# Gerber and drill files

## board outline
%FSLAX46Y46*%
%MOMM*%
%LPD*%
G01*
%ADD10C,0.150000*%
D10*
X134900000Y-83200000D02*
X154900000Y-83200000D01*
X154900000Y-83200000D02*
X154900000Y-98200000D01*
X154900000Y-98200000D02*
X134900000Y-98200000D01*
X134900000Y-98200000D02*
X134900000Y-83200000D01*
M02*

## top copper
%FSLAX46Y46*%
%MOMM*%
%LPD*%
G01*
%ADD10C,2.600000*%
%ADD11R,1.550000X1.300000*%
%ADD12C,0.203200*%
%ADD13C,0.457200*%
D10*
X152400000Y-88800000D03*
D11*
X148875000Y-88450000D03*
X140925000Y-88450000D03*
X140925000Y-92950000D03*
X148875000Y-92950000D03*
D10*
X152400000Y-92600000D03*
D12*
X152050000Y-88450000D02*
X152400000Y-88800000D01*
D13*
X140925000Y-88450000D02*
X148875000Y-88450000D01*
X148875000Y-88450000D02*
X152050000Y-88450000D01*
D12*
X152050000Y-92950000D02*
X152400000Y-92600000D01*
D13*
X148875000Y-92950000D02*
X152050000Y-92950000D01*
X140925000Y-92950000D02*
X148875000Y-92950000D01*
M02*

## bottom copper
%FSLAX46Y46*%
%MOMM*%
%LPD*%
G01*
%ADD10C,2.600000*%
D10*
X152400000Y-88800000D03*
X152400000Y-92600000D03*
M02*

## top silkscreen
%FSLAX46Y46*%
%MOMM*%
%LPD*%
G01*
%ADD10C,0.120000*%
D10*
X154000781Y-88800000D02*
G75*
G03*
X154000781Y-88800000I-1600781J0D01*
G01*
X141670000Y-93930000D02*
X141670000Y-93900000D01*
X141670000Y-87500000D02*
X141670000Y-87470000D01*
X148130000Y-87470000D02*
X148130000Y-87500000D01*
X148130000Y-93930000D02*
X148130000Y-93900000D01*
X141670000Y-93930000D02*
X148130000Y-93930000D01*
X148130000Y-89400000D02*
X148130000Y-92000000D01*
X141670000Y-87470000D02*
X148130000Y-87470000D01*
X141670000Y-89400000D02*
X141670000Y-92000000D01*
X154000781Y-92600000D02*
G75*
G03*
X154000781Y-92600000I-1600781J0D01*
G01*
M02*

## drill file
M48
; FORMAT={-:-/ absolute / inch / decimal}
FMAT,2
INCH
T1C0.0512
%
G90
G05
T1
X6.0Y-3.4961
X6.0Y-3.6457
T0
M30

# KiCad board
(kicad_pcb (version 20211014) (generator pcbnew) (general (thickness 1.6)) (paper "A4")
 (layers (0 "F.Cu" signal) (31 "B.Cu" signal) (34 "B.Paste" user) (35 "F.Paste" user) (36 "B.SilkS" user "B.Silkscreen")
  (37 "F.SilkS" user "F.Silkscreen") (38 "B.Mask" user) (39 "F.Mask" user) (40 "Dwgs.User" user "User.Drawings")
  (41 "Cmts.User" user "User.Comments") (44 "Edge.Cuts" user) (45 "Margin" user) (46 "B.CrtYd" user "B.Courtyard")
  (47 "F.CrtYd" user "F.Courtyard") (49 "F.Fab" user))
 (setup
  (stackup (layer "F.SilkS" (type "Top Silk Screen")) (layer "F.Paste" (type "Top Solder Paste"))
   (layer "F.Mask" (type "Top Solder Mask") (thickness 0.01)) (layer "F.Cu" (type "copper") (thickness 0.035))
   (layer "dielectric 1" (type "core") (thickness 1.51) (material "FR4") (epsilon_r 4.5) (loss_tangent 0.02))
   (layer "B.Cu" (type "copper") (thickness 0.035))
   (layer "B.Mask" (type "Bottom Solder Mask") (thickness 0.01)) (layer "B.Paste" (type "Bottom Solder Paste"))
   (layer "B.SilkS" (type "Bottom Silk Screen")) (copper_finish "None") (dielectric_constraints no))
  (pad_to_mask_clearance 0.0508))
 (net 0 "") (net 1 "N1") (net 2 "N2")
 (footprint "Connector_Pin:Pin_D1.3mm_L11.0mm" (layer "F.Cu") (at 152.4 88.8)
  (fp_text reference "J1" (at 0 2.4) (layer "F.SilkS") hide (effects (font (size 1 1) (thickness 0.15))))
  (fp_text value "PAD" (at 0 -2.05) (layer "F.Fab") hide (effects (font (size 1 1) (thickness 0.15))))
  (fp_circle (center 0 0) (end 1.6 0.05) (layer "F.SilkS") (width 0.12) (fill none))
  (pad "1" thru_hole circle (at 0 0) (size 2.6 2.6) (drill 1.3) (layers *.Cu *.Mask) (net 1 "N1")))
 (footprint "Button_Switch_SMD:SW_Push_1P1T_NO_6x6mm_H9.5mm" (layer "F.Cu") (at 144.9 90.7)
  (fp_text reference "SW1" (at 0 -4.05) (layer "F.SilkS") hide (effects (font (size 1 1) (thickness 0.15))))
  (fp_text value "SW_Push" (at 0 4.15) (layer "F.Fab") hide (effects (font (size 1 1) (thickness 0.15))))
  (fp_line (start -3.23 3.23) (end -3.23 3.2) (layer "F.SilkS") (width 0.12))
  (fp_line (start -3.23 -3.2) (end -3.23 -3.23) (layer "F.SilkS") (width 0.12))
  (fp_line (start 3.23 -3.23) (end 3.23 -3.2) (layer "F.SilkS") (width 0.12))
  (fp_line (start 3.23 3.23) (end 3.23 3.2) (layer "F.SilkS") (width 0.12))
  (fp_line (start -3.23 3.23) (end 3.23 3.23) (layer "F.SilkS") (width 0.12))
  (fp_line (start 3.23 -1.3) (end 3.23 1.3) (layer "F.SilkS") (width 0.12))
  (fp_line (start -3.23 -3.23) (end 3.23 -3.23) (layer "F.SilkS") (width 0.12))
  (fp_line (start -3.23 -1.3) (end -3.23 1.3) (layer "F.SilkS") (width 0.12))
  (pad "1" smd rect (at 3.975 -2.25) (size 1.55 1.3) (layers "F.Cu" "F.Paste" "F.Mask") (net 1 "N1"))
  (pad "1" smd rect (at -3.975 -2.25) (size 1.55 1.3) (layers "F.Cu" "F.Paste" "F.Mask") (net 1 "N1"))
  (pad "2" smd rect (at -3.975 2.25) (size 1.55 1.3) (layers "F.Cu" "F.Paste" "F.Mask") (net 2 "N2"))
  (pad "2" smd rect (at 3.975 2.25) (size 1.55 1.3) (layers "F.Cu" "F.Paste" "F.Mask") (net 2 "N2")))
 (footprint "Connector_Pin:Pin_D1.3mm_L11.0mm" (layer "F.Cu") (at 152.4 92.6)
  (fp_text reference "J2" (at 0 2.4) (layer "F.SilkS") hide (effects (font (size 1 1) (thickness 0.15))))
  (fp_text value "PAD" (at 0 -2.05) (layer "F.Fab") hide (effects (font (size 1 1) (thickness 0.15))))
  (fp_circle (center 0 0) (end 1.6 0.05) (layer "F.SilkS") (width 0.12) (fill none))
  (pad "1" thru_hole circle (at 0 0) (size 2.6 2.6) (drill 1.3) (layers *.Cu *.Mask) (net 2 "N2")))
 (gr_rect (start 134.9 83.2) (end 154.9 98.2) (layer "Edge.Cuts") (width 0.15) (fill none))
 (segment (start 152.05 88.45) (end 152.4 88.8) (width 0.2032) (layer "F.Cu") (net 1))
 (segment (start 140.925 88.45) (end 148.875 88.45) (width 0.4572) (layer "F.Cu") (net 1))
 (segment (start 148.875 88.45) (end 152.05 88.45) (width 0.4572) (layer "F.Cu") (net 1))
 (segment (start 152.05 92.95) (end 152.4 92.6) (width 0.2032) (layer "F.Cu") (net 2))
 (segment (start 148.875 92.95) (end 152.05 92.95) (width 0.4572) (layer "F.Cu") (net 2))
 (segment (start 140.925 92.95) (end 148.875 92.95) (width 0.4572) (layer "F.Cu") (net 2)))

